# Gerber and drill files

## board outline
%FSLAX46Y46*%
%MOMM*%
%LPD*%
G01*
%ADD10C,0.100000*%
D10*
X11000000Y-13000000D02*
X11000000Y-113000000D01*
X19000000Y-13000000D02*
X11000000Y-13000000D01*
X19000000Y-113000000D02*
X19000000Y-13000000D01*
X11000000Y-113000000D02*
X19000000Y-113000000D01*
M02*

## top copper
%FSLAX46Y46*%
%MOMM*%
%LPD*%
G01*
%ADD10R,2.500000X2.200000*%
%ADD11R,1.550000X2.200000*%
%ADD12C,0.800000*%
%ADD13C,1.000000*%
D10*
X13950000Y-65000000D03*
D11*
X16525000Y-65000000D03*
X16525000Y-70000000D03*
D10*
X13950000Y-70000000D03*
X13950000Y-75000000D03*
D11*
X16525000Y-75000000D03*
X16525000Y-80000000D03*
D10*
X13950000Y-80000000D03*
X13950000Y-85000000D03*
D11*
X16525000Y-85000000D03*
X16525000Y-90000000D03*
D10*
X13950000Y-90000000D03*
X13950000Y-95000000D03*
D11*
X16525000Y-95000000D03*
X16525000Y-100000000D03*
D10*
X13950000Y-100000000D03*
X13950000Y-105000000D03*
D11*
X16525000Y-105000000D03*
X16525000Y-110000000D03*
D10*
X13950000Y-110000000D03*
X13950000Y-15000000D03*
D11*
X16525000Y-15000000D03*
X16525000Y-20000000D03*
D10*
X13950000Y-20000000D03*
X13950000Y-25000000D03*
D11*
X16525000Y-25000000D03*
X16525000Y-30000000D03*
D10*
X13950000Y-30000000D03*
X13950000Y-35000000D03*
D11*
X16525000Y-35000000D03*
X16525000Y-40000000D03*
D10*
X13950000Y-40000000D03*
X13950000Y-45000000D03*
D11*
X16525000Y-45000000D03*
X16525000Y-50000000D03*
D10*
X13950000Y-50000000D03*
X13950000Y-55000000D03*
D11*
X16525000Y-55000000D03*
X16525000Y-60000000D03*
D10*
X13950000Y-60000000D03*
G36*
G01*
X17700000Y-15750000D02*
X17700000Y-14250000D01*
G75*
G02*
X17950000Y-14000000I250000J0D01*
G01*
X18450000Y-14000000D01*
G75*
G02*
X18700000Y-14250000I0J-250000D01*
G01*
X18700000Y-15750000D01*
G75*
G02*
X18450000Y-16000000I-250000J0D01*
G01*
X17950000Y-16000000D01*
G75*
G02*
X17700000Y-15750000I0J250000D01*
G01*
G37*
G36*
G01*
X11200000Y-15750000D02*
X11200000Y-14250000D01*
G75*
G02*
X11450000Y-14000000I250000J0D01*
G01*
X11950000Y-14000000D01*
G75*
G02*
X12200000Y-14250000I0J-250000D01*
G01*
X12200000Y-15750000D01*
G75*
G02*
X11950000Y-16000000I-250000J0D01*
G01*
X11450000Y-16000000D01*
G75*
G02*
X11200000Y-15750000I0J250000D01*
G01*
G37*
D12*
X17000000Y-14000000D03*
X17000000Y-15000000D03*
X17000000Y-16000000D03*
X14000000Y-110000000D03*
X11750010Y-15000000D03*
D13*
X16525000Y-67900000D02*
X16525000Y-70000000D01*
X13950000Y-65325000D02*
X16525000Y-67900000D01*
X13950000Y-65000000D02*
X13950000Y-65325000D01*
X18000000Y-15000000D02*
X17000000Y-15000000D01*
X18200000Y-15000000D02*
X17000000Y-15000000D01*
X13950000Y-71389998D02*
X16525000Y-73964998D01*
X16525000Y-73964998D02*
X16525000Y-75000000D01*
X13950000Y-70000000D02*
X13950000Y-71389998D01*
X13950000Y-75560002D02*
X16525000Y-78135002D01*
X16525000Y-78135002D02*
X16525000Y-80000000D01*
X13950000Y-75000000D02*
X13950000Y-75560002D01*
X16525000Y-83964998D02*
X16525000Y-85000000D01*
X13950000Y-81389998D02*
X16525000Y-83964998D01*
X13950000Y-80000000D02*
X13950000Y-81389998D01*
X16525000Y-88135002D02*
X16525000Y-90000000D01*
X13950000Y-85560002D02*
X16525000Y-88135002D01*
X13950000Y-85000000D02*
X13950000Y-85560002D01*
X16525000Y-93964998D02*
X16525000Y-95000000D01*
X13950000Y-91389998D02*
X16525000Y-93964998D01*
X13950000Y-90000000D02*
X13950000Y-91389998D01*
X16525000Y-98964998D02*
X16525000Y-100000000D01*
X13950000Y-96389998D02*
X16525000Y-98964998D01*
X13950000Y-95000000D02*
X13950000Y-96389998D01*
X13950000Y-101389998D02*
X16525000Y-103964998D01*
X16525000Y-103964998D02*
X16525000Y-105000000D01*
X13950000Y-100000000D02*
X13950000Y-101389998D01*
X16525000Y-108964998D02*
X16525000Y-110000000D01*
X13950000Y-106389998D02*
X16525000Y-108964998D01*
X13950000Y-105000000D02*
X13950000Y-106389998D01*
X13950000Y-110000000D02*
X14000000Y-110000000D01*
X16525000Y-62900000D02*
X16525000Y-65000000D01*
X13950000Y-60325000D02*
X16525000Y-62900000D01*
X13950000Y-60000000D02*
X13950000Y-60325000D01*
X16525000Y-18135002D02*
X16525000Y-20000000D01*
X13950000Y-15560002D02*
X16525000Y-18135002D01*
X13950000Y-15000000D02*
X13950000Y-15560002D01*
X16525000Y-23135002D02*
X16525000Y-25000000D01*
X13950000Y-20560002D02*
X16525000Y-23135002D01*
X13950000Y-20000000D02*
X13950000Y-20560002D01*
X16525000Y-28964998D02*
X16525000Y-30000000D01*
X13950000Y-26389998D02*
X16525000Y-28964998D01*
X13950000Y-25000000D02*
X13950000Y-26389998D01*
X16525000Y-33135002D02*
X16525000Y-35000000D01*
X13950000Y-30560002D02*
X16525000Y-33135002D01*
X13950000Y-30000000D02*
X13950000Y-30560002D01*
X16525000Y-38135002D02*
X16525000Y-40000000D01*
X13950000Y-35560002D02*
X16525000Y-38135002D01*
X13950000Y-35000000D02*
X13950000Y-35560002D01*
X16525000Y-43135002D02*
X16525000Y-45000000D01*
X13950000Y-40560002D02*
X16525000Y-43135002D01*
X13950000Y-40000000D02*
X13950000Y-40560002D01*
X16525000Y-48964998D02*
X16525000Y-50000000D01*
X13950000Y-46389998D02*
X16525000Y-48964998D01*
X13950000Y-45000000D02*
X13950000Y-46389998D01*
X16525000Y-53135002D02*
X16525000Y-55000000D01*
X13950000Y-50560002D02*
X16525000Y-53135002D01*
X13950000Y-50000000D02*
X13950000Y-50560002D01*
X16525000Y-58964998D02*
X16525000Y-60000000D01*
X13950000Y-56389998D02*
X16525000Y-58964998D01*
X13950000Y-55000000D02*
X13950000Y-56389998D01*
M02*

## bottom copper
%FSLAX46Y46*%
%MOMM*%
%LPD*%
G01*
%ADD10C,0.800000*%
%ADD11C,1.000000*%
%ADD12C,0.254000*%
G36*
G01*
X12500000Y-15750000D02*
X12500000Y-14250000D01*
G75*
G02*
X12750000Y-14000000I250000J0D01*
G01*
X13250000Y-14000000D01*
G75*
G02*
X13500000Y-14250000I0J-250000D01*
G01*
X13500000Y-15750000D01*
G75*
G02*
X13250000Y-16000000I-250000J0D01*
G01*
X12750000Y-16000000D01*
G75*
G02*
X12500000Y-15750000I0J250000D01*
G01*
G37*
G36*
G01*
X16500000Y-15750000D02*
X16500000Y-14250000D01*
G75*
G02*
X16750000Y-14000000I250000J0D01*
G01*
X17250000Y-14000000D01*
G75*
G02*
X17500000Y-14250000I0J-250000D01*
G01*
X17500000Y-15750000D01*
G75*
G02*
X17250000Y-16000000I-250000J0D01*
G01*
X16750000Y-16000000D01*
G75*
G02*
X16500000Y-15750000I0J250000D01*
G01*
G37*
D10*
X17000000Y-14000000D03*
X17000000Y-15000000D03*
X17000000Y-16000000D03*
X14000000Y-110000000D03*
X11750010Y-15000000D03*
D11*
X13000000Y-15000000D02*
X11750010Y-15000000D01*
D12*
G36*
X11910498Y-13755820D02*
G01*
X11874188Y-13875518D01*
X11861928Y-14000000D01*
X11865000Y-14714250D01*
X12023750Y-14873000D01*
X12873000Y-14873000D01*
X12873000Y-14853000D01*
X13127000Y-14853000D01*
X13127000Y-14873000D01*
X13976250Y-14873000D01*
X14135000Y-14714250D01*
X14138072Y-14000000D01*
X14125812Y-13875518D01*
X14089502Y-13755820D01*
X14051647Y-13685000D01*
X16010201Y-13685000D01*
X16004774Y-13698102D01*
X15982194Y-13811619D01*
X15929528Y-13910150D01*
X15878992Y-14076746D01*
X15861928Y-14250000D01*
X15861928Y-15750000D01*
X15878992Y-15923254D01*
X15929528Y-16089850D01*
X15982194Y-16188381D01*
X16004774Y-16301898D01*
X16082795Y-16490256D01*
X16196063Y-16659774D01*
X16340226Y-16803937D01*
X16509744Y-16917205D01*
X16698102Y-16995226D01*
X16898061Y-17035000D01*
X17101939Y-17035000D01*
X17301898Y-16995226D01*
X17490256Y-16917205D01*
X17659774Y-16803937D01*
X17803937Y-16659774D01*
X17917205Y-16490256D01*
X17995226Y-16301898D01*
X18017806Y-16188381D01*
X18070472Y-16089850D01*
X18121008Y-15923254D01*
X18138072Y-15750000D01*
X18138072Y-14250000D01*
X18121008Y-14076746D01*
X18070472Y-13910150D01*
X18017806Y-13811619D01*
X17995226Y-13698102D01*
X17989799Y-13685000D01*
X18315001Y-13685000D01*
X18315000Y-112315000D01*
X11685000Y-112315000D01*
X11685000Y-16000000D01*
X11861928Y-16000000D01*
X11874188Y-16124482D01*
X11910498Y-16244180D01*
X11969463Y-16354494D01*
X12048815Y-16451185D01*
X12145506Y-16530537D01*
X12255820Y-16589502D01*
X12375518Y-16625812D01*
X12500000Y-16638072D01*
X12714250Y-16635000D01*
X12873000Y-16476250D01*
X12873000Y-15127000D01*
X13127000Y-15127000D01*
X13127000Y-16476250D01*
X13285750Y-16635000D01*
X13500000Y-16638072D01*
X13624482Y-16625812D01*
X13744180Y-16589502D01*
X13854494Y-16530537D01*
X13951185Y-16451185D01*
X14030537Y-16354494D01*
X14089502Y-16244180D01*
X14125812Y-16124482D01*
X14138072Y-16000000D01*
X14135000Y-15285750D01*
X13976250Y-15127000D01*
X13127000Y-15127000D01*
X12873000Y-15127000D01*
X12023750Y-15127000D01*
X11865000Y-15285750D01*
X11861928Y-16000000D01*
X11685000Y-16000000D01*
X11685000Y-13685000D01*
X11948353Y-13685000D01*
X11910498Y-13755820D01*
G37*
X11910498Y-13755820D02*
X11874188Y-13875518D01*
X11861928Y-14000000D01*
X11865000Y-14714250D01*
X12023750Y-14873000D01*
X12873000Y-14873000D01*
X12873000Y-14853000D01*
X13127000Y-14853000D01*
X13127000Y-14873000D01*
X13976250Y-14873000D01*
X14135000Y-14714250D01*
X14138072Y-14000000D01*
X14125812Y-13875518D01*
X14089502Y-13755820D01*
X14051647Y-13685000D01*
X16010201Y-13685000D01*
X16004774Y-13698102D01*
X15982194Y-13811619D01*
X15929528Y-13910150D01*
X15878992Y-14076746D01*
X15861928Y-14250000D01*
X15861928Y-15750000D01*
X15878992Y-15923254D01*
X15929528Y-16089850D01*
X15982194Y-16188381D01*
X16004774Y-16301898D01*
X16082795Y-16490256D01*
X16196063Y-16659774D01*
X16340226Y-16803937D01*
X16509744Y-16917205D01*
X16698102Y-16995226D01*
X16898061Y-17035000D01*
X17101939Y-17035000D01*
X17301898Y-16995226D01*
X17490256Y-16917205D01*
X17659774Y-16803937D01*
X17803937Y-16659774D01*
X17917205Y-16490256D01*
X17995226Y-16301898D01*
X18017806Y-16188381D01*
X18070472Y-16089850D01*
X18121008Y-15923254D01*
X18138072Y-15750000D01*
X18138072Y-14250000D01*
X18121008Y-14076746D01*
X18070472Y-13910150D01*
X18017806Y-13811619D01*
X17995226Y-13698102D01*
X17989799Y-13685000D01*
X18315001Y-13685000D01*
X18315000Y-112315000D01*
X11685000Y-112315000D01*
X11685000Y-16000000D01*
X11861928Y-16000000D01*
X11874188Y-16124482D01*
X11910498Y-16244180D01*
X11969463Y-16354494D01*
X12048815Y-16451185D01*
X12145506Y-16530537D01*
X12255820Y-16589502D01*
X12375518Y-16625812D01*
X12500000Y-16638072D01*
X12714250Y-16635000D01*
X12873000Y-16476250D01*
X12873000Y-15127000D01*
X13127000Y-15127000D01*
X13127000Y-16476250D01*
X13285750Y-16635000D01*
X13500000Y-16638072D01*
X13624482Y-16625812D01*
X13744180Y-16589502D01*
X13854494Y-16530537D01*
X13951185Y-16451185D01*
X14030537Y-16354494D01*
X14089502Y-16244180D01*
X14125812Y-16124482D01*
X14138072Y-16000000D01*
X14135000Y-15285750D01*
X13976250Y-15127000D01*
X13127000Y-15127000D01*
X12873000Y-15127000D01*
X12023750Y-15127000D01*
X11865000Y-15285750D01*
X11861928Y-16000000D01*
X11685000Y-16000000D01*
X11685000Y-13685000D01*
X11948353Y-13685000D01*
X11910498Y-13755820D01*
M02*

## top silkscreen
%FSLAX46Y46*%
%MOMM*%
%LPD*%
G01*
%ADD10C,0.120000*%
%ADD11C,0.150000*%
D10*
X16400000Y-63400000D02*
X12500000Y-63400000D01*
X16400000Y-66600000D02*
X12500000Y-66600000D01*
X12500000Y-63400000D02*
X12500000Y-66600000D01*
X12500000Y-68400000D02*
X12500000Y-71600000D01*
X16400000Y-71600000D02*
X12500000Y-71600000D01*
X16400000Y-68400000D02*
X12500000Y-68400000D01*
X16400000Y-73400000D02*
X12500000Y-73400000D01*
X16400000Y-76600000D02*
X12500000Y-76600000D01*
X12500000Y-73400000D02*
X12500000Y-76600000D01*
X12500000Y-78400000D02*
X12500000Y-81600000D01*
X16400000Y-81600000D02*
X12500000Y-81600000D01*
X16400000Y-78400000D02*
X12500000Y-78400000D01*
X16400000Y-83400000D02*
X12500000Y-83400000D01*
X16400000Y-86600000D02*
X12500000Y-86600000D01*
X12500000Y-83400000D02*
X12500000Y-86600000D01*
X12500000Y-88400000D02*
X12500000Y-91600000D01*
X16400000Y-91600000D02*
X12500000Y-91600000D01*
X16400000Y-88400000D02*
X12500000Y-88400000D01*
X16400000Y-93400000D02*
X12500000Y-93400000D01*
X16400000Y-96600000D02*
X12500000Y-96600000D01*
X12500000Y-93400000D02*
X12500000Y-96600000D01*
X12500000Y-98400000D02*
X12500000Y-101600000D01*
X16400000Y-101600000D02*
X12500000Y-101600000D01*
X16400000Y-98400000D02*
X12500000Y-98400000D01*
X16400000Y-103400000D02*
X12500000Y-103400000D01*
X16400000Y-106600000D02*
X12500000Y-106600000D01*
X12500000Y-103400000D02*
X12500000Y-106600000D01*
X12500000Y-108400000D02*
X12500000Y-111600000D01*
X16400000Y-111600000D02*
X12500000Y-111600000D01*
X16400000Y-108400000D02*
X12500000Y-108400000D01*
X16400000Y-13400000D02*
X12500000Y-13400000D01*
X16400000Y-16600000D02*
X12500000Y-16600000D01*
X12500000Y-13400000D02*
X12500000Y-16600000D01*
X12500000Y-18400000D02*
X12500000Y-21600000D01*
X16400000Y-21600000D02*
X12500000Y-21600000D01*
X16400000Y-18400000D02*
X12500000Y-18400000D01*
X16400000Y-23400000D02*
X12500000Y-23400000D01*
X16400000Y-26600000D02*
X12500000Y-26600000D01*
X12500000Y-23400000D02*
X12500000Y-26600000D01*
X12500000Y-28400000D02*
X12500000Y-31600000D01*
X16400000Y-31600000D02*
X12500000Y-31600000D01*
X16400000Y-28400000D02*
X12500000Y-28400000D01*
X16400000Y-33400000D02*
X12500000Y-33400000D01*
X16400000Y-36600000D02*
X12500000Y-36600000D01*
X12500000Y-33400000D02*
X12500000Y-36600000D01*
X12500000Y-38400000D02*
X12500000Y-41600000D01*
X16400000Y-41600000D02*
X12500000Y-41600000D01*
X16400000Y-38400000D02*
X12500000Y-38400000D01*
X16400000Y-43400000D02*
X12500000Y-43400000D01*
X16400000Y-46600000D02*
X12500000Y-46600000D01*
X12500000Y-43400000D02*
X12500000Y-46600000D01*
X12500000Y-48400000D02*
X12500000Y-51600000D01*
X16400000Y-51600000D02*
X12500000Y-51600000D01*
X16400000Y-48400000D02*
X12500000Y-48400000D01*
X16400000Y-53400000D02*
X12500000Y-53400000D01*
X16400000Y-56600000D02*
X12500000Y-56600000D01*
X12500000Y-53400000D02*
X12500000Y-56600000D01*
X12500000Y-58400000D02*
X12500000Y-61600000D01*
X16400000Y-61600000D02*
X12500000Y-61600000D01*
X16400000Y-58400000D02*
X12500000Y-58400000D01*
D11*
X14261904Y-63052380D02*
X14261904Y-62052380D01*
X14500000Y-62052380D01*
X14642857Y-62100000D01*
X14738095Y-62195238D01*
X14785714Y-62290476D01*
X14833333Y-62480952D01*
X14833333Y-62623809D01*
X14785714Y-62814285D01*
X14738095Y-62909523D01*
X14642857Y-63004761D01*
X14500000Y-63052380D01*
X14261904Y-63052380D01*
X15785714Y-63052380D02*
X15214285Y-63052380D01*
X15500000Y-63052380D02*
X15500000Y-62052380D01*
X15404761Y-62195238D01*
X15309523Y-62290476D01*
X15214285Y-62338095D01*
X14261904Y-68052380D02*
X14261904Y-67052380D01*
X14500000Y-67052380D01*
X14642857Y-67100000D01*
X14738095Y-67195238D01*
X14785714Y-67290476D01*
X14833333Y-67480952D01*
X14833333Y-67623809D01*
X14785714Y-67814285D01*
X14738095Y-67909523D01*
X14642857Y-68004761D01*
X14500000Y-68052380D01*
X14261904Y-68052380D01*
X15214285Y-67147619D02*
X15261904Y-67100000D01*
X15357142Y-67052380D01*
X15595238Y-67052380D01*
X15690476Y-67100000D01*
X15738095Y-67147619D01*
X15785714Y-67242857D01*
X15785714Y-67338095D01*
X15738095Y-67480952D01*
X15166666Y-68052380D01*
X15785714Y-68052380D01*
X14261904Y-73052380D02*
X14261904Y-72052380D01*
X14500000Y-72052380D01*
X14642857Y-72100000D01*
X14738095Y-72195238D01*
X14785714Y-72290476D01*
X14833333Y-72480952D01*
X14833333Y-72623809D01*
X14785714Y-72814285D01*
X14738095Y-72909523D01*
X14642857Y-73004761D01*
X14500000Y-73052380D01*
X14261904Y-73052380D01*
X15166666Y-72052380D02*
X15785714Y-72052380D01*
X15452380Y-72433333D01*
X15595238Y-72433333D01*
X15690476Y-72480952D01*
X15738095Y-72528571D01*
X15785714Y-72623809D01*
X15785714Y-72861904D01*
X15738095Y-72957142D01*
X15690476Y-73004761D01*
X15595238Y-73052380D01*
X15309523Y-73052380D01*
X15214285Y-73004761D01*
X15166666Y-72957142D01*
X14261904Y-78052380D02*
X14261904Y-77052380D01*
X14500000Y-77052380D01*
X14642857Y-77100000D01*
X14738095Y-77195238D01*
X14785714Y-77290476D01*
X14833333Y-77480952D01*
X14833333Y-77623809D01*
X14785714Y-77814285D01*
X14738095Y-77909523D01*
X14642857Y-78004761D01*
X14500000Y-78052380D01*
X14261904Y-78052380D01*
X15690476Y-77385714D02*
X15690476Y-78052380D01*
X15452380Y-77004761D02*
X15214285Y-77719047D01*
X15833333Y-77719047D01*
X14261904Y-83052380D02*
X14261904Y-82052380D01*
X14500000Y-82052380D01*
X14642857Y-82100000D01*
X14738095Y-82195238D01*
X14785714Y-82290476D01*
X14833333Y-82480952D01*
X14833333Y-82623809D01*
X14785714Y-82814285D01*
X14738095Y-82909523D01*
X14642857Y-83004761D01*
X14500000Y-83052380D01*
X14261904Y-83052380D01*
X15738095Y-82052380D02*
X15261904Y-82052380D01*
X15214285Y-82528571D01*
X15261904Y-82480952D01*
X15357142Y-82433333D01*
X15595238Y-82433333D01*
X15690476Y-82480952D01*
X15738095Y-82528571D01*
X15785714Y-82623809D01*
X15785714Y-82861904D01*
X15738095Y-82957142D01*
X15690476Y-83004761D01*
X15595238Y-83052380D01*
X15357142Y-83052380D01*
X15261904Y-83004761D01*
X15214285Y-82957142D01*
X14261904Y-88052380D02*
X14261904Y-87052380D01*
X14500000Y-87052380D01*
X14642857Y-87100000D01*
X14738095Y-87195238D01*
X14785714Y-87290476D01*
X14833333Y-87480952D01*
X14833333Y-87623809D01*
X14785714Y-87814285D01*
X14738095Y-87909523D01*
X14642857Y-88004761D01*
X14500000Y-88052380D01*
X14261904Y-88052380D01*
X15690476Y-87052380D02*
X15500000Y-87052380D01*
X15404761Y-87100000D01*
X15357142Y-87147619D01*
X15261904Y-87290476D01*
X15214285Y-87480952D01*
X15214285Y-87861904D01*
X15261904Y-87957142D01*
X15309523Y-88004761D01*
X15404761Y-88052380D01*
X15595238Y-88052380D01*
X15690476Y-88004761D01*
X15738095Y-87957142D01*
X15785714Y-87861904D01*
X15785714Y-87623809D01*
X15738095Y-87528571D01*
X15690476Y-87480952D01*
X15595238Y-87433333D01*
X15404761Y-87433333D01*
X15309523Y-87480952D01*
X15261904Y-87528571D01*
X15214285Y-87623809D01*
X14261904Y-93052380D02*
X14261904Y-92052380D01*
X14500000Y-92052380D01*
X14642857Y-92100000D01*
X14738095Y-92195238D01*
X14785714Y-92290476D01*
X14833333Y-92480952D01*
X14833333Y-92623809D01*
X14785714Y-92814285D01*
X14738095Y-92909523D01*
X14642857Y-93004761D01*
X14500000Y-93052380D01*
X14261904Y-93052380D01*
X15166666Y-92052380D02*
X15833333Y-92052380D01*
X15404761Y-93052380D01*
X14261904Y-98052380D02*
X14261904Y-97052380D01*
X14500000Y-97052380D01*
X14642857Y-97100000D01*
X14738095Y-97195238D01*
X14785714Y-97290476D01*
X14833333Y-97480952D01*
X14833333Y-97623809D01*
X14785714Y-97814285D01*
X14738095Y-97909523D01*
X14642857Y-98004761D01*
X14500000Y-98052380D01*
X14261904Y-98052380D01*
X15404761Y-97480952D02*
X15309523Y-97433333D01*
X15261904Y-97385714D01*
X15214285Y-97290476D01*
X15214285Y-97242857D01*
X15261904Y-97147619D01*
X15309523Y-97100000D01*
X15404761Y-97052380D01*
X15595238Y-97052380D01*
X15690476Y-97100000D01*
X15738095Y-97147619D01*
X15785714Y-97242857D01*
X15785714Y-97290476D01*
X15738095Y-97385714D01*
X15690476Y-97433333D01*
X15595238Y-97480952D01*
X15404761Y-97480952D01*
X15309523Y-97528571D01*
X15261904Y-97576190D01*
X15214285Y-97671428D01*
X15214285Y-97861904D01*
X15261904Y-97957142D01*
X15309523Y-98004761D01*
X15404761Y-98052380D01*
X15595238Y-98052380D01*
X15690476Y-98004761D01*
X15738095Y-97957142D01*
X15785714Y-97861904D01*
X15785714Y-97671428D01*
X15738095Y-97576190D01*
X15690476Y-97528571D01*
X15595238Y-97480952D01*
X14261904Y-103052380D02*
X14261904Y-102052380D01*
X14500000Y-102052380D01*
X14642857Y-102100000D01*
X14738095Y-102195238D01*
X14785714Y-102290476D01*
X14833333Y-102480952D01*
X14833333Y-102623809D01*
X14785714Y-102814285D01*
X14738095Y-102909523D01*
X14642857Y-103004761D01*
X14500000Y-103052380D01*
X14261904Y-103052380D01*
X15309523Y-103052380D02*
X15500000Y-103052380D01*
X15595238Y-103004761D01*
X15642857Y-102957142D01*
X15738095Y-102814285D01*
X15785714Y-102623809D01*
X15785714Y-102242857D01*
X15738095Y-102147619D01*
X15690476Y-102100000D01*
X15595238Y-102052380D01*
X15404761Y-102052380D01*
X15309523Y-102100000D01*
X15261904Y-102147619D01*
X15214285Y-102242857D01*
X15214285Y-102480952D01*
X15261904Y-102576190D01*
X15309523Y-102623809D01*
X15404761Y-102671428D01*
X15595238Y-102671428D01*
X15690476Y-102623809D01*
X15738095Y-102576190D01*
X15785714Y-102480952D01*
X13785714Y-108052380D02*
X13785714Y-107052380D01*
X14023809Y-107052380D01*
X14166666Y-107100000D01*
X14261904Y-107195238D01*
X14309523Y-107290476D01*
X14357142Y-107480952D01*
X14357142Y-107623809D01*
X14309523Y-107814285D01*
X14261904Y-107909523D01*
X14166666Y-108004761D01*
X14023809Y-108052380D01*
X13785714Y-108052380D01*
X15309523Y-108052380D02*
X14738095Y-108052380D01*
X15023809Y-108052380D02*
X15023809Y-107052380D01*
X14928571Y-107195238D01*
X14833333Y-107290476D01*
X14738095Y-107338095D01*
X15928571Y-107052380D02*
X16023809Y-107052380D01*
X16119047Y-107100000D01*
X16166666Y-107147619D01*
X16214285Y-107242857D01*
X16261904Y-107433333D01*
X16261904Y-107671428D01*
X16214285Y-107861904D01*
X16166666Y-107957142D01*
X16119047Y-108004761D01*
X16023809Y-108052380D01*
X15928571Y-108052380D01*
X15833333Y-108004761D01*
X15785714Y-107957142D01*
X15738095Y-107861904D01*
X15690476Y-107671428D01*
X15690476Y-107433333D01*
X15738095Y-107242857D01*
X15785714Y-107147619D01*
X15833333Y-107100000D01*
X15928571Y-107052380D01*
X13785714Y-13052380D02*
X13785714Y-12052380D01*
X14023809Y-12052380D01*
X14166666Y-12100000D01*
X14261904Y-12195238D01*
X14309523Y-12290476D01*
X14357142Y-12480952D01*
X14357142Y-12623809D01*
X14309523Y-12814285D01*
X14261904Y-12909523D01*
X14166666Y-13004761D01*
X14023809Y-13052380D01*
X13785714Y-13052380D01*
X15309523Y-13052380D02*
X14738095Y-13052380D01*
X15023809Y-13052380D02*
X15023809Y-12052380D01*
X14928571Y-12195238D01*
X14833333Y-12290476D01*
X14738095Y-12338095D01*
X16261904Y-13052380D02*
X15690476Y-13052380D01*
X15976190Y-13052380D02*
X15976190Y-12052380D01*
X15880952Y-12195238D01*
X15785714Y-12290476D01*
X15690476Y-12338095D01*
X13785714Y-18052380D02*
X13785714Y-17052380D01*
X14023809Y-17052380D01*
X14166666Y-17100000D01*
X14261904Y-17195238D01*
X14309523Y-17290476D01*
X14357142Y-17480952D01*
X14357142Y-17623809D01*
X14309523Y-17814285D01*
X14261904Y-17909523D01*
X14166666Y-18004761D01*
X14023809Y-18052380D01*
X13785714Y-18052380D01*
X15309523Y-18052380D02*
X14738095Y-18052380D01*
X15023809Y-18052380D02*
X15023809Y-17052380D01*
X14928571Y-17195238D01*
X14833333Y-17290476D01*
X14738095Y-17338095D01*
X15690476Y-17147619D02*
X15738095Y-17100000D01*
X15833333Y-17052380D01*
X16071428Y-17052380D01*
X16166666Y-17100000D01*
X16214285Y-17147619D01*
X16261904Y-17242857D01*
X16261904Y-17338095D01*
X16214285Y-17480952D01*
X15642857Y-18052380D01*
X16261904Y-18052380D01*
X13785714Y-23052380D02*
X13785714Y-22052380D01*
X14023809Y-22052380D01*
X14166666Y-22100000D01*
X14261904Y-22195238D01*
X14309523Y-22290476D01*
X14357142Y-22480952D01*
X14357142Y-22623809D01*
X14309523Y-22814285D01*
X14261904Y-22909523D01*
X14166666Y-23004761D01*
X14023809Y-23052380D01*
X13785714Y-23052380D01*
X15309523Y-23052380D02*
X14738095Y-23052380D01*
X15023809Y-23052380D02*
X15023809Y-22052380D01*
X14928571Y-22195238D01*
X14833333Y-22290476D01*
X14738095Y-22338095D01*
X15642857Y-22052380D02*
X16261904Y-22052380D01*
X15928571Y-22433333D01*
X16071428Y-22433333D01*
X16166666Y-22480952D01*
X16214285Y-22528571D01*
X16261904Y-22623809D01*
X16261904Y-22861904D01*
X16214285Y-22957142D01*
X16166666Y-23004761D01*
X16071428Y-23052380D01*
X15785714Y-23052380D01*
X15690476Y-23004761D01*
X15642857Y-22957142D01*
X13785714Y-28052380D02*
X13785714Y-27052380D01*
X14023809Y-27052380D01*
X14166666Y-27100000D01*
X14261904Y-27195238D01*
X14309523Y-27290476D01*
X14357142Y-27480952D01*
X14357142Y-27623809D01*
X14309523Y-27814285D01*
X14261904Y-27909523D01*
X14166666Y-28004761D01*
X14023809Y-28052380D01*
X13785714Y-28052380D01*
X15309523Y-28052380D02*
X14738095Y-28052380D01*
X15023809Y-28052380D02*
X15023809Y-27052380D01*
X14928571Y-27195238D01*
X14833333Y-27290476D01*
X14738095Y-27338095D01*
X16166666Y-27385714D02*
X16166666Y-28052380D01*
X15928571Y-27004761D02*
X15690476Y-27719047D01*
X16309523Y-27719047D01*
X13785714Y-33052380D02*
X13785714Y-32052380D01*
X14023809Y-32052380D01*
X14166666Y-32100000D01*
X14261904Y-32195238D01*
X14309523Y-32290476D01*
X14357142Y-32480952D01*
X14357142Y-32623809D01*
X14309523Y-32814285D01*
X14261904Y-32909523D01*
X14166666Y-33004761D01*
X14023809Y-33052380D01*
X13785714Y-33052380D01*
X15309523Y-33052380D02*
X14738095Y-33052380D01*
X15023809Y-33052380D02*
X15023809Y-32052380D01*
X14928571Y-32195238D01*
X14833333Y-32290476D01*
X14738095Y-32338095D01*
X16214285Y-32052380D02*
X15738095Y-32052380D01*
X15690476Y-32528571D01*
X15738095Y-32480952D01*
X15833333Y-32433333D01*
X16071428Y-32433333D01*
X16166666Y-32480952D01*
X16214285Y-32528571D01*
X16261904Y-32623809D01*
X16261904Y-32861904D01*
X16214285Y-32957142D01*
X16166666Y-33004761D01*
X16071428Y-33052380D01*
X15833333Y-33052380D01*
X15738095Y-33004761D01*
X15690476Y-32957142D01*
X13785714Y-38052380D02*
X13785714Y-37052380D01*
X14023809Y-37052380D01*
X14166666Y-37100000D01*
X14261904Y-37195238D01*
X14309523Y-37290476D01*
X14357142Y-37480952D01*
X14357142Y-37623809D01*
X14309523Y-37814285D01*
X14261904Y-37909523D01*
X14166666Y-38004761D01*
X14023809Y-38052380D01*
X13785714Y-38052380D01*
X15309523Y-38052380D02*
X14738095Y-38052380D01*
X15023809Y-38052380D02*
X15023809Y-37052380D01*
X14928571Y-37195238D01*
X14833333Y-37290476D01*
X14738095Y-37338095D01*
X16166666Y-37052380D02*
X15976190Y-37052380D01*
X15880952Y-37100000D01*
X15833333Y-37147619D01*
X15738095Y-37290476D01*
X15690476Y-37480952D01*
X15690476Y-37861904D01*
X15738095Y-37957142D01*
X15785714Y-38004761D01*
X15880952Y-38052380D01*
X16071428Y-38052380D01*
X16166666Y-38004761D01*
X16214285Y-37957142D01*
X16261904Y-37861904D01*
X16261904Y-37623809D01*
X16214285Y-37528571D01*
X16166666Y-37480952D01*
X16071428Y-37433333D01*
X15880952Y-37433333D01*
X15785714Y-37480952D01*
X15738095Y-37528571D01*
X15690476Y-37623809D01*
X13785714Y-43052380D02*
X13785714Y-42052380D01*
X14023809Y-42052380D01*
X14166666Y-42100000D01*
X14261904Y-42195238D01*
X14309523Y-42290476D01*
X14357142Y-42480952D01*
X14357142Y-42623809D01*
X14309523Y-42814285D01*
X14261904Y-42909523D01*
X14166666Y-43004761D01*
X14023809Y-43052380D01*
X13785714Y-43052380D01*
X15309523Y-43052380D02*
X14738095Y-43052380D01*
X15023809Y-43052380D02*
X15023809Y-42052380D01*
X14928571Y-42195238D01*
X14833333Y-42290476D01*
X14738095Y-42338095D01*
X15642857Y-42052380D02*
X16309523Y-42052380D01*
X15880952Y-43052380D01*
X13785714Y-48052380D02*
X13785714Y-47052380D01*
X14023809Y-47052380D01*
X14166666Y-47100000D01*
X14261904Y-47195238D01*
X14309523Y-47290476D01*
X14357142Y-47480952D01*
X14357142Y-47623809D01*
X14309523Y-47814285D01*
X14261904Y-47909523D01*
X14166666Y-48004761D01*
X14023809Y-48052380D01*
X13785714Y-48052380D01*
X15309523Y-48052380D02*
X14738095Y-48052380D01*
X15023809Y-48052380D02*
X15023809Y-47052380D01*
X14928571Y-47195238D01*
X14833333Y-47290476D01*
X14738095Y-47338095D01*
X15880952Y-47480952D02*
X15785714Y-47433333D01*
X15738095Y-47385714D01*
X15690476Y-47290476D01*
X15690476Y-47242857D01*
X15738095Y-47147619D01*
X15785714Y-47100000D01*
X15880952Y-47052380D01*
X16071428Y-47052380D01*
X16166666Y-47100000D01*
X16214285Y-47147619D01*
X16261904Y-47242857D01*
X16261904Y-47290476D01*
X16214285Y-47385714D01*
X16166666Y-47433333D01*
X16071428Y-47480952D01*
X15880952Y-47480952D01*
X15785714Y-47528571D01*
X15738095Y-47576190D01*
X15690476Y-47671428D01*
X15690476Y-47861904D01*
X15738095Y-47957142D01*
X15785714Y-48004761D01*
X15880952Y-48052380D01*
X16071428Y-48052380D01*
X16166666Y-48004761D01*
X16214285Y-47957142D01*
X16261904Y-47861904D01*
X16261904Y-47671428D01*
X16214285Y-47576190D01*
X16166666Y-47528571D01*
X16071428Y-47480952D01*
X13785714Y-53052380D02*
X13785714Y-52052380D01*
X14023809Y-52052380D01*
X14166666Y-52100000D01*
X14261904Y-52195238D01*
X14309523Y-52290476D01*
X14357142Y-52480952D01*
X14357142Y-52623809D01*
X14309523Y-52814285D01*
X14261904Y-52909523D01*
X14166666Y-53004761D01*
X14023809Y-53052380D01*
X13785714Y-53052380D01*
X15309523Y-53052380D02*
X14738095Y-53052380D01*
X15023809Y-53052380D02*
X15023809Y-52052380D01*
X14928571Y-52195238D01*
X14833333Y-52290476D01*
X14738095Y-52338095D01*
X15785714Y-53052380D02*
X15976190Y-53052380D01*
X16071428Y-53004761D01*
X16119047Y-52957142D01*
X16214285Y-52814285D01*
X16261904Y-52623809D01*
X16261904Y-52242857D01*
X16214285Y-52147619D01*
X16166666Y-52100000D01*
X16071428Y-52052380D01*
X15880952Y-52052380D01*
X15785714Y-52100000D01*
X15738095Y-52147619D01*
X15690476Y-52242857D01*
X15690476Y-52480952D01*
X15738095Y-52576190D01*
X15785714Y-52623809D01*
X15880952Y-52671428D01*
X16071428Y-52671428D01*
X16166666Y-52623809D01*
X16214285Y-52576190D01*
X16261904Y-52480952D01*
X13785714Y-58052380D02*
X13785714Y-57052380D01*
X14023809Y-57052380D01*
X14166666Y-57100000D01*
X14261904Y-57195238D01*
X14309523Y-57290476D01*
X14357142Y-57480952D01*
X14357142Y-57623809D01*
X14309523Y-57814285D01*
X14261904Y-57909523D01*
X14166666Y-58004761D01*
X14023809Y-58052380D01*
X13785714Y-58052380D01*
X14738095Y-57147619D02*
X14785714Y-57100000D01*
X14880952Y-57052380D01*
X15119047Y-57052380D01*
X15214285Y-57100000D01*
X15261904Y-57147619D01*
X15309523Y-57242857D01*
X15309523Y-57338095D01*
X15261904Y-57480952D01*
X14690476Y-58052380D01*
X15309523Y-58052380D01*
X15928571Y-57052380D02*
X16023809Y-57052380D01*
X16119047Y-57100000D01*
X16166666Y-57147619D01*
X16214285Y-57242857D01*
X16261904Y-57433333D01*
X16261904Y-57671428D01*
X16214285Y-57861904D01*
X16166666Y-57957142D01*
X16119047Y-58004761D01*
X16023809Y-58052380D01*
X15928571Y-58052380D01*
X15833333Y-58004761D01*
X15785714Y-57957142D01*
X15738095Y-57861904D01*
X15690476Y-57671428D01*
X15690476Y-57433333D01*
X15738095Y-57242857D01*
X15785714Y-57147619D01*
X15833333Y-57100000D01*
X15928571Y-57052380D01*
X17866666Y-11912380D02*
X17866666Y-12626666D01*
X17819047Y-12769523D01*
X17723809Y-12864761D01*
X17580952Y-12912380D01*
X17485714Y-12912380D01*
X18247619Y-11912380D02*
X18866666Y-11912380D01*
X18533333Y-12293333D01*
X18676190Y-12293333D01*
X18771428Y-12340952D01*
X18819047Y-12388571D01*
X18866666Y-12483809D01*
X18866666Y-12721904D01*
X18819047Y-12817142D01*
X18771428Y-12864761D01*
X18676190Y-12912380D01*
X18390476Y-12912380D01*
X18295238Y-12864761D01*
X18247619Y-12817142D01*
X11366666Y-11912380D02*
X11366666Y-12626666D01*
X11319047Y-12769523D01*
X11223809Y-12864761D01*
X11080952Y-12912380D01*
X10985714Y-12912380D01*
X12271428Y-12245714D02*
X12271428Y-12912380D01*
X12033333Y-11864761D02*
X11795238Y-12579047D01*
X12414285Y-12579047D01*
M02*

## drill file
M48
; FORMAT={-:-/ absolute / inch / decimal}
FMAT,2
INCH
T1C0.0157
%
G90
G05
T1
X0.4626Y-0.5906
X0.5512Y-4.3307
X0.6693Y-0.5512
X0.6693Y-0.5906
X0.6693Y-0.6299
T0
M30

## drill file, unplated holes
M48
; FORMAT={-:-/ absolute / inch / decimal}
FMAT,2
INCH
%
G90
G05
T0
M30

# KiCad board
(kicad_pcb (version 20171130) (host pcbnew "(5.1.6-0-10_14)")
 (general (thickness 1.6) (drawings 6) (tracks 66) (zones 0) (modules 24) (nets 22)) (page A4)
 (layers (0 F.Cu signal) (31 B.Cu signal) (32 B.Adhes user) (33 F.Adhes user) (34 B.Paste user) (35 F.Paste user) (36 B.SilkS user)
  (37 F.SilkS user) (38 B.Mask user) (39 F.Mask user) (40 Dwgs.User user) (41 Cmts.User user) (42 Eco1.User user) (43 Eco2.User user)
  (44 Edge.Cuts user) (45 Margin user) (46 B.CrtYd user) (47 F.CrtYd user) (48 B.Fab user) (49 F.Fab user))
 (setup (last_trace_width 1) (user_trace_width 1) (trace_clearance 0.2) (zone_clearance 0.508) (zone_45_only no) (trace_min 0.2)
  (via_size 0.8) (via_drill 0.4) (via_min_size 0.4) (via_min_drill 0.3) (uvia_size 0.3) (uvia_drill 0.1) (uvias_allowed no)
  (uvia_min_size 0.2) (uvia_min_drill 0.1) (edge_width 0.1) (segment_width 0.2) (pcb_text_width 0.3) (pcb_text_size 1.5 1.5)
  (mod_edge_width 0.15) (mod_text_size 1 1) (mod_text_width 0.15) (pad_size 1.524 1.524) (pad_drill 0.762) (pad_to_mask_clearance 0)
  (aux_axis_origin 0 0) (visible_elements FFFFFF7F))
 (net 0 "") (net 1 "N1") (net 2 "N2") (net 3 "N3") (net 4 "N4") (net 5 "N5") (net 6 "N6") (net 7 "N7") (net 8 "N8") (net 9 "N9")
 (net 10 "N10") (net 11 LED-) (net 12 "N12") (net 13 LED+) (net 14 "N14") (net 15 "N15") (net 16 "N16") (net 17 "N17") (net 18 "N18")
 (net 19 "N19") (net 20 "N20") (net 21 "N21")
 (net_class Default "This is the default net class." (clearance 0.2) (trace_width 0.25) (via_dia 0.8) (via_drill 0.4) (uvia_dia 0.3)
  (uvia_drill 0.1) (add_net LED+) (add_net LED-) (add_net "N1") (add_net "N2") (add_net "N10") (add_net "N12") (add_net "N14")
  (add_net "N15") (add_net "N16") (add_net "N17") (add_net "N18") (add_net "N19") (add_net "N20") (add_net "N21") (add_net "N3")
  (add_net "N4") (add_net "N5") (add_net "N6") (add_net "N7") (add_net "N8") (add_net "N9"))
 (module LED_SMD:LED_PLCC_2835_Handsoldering (layer F.Cu) (at 15 65)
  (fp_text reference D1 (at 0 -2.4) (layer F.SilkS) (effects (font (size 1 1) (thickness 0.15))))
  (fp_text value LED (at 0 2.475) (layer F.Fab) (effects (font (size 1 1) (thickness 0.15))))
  (fp_line (start 1.4 -1.6) (end -2.5 -1.6) (layer F.SilkS) (width 0.12))
  (fp_line (start 1.4 1.6) (end -2.5 1.6) (layer F.SilkS) (width 0.12))
  (fp_line (start -2.5 -1.6) (end -2.5 1.6) (layer F.SilkS) (width 0.12))
  (pad 1 smd rect (at -1.05 0) (size 2.5 2.2) (layers F.Cu F.Paste F.Mask) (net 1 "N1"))
  (pad 2 smd rect (at 1.525 0) (size 1.55 2.2) (layers F.Cu F.Paste F.Mask) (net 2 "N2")))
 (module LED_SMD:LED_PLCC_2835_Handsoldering (layer F.Cu) (at 15 70)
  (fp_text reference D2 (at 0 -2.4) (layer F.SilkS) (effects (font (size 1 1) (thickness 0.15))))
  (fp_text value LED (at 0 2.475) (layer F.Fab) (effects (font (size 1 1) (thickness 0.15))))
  (fp_line (start -2.5 -1.6) (end -2.5 1.6) (layer F.SilkS) (width 0.12))
  (fp_line (start 1.4 1.6) (end -2.5 1.6) (layer F.SilkS) (width 0.12))
  (fp_line (start 1.4 -1.6) (end -2.5 -1.6) (layer F.SilkS) (width 0.12))
  (pad 2 smd rect (at 1.525 0) (size 1.55 2.2) (layers F.Cu F.Paste F.Mask) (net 1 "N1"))
  (pad 1 smd rect (at -1.05 0) (size 2.5 2.2) (layers F.Cu F.Paste F.Mask) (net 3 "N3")))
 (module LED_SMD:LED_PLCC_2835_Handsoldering (layer F.Cu) (at 15 75)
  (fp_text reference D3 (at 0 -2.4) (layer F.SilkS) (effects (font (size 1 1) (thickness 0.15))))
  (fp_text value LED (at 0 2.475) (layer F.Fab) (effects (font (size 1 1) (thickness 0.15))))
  (fp_line (start 1.4 -1.6) (end -2.5 -1.6) (layer F.SilkS) (width 0.12))
  (fp_line (start 1.4 1.6) (end -2.5 1.6) (layer F.SilkS) (width 0.12))
  (fp_line (start -2.5 -1.6) (end -2.5 1.6) (layer F.SilkS) (width 0.12))
  (pad 1 smd rect (at -1.05 0) (size 2.5 2.2) (layers F.Cu F.Paste F.Mask) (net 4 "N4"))
  (pad 2 smd rect (at 1.525 0) (size 1.55 2.2) (layers F.Cu F.Paste F.Mask) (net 3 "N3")))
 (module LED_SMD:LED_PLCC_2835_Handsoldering (layer F.Cu) (at 15 80)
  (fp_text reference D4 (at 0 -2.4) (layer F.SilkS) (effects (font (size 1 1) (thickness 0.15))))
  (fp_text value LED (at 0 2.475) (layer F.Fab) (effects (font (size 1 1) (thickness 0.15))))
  (fp_line (start -2.5 -1.6) (end -2.5 1.6) (layer F.SilkS) (width 0.12))
  (fp_line (start 1.4 1.6) (end -2.5 1.6) (layer F.SilkS) (width 0.12))
  (fp_line (start 1.4 -1.6) (end -2.5 -1.6) (layer F.SilkS) (width 0.12))
  (pad 2 smd rect (at 1.525 0) (size 1.55 2.2) (layers F.Cu F.Paste F.Mask) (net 4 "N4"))
  (pad 1 smd rect (at -1.05 0) (size 2.5 2.2) (layers F.Cu F.Paste F.Mask) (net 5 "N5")))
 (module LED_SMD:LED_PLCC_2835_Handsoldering (layer F.Cu) (at 15 85)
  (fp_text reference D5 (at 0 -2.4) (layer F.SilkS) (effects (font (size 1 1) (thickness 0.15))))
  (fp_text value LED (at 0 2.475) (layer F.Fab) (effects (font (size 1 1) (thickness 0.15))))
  (fp_line (start 1.4 -1.6) (end -2.5 -1.6) (layer F.SilkS) (width 0.12))
  (fp_line (start 1.4 1.6) (end -2.5 1.6) (layer F.SilkS) (width 0.12))
  (fp_line (start -2.5 -1.6) (end -2.5 1.6) (layer F.SilkS) (width 0.12))
  (pad 1 smd rect (at -1.05 0) (size 2.5 2.2) (layers F.Cu F.Paste F.Mask) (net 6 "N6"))
  (pad 2 smd rect (at 1.525 0) (size 1.55 2.2) (layers F.Cu F.Paste F.Mask) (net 5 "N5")))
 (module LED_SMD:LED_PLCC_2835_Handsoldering (layer F.Cu) (at 15 90)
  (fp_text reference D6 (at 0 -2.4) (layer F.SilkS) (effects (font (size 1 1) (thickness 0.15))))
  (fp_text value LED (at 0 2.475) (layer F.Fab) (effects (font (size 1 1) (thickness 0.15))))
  (fp_line (start -2.5 -1.6) (end -2.5 1.6) (layer F.SilkS) (width 0.12))
  (fp_line (start 1.4 1.6) (end -2.5 1.6) (layer F.SilkS) (width 0.12))
  (fp_line (start 1.4 -1.6) (end -2.5 -1.6) (layer F.SilkS) (width 0.12))
  (pad 2 smd rect (at 1.525 0) (size 1.55 2.2) (layers F.Cu F.Paste F.Mask) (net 6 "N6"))
  (pad 1 smd rect (at -1.05 0) (size 2.5 2.2) (layers F.Cu F.Paste F.Mask) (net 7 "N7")))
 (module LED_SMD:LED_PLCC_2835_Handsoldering (layer F.Cu) (at 15 95)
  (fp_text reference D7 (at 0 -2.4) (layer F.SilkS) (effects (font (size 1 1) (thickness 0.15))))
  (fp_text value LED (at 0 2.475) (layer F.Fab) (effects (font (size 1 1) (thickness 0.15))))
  (fp_line (start 1.4 -1.6) (end -2.5 -1.6) (layer F.SilkS) (width 0.12))
  (fp_line (start 1.4 1.6) (end -2.5 1.6) (layer F.SilkS) (width 0.12))
  (fp_line (start -2.5 -1.6) (end -2.5 1.6) (layer F.SilkS) (width 0.12))
  (pad 1 smd rect (at -1.05 0) (size 2.5 2.2) (layers F.Cu F.Paste F.Mask) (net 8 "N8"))
  (pad 2 smd rect (at 1.525 0) (size 1.55 2.2) (layers F.Cu F.Paste F.Mask) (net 7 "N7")))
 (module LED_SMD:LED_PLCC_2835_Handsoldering (layer F.Cu) (at 15 100)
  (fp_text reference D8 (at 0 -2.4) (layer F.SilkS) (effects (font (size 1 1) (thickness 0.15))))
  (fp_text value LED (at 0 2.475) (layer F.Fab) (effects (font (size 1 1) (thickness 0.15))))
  (fp_line (start -2.5 -1.6) (end -2.5 1.6) (layer F.SilkS) (width 0.12))
  (fp_line (start 1.4 1.6) (end -2.5 1.6) (layer F.SilkS) (width 0.12))
  (fp_line (start 1.4 -1.6) (end -2.5 -1.6) (layer F.SilkS) (width 0.12))
  (pad 2 smd rect (at 1.525 0) (size 1.55 2.2) (layers F.Cu F.Paste F.Mask) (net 8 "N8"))
  (pad 1 smd rect (at -1.05 0) (size 2.5 2.2) (layers F.Cu F.Paste F.Mask) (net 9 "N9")))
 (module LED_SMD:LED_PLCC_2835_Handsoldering (layer F.Cu) (at 15 105)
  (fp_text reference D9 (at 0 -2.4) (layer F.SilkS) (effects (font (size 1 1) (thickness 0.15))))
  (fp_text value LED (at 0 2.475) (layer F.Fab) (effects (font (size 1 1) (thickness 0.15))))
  (fp_line (start 1.4 -1.6) (end -2.5 -1.6) (layer F.SilkS) (width 0.12))
  (fp_line (start 1.4 1.6) (end -2.5 1.6) (layer F.SilkS) (width 0.12))
  (fp_line (start -2.5 -1.6) (end -2.5 1.6) (layer F.SilkS) (width 0.12))
  (pad 1 smd rect (at -1.05 0) (size 2.5 2.2) (layers F.Cu F.Paste F.Mask) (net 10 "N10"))
  (pad 2 smd rect (at 1.525 0) (size 1.55 2.2) (layers F.Cu F.Paste F.Mask) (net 9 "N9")))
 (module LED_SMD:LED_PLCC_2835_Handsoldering (layer F.Cu) (at 15 110)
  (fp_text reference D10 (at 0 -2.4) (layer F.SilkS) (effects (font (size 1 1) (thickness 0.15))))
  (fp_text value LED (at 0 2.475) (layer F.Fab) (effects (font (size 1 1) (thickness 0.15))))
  (fp_line (start -2.5 -1.6) (end -2.5 1.6) (layer F.SilkS) (width 0.12))
  (fp_line (start 1.4 1.6) (end -2.5 1.6) (layer F.SilkS) (width 0.12))
  (fp_line (start 1.4 -1.6) (end -2.5 -1.6) (layer F.SilkS) (width 0.12))
  (pad 2 smd rect (at 1.525 0) (size 1.55 2.2) (layers F.Cu F.Paste F.Mask) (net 10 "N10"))
  (pad 1 smd rect (at -1.05 0) (size 2.5 2.2) (layers F.Cu F.Paste F.Mask) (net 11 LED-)))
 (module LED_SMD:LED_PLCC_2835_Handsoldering (layer F.Cu) (at 15 15)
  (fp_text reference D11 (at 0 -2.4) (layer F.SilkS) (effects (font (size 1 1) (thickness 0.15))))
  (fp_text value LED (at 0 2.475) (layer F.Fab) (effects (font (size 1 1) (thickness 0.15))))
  (fp_line (start 1.4 -1.6) (end -2.5 -1.6) (layer F.SilkS) (width 0.12))
  (fp_line (start 1.4 1.6) (end -2.5 1.6) (layer F.SilkS) (width 0.12))
  (fp_line (start -2.5 -1.6) (end -2.5 1.6) (layer F.SilkS) (width 0.12))
  (pad 1 smd rect (at -1.05 0) (size 2.5 2.2) (layers F.Cu F.Paste F.Mask) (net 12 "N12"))
  (pad 2 smd rect (at 1.525 0) (size 1.55 2.2) (layers F.Cu F.Paste F.Mask) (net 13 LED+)))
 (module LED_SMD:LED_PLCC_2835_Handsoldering (layer F.Cu) (at 15 20)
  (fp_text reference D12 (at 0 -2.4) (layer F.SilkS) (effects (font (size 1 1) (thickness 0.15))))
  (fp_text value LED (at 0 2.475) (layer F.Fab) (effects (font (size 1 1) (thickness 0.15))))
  (fp_line (start -2.5 -1.6) (end -2.5 1.6) (layer F.SilkS) (width 0.12))
  (fp_line (start 1.4 1.6) (end -2.5 1.6) (layer F.SilkS) (width 0.12))
  (fp_line (start 1.4 -1.6) (end -2.5 -1.6) (layer F.SilkS) (width 0.12))
  (pad 2 smd rect (at 1.525 0) (size 1.55 2.2) (layers F.Cu F.Paste F.Mask) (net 12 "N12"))
  (pad 1 smd rect (at -1.05 0) (size 2.5 2.2) (layers F.Cu F.Paste F.Mask) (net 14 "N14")))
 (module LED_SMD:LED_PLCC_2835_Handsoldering (layer F.Cu) (at 15 25)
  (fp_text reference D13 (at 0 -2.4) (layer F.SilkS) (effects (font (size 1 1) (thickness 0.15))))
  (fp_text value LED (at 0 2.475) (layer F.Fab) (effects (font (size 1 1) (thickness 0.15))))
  (fp_line (start 1.4 -1.6) (end -2.5 -1.6) (layer F.SilkS) (width 0.12))
  (fp_line (start 1.4 1.6) (end -2.5 1.6) (layer F.SilkS) (width 0.12))
  (fp_line (start -2.5 -1.6) (end -2.5 1.6) (layer F.SilkS) (width 0.12))
  (pad 1 smd rect (at -1.05 0) (size 2.5 2.2) (layers F.Cu F.Paste F.Mask) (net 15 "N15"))
  (pad 2 smd rect (at 1.525 0) (size 1.55 2.2) (layers F.Cu F.Paste F.Mask) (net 14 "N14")))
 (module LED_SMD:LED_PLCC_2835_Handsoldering (layer F.Cu) (at 15 30)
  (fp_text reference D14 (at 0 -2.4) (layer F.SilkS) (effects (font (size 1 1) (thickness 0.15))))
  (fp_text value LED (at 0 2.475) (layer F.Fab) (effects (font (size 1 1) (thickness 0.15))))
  (fp_line (start -2.5 -1.6) (end -2.5 1.6) (layer F.SilkS) (width 0.12))
  (fp_line (start 1.4 1.6) (end -2.5 1.6) (layer F.SilkS) (width 0.12))
  (fp_line (start 1.4 -1.6) (end -2.5 -1.6) (layer F.SilkS) (width 0.12))
  (pad 2 smd rect (at 1.525 0) (size 1.55 2.2) (layers F.Cu F.Paste F.Mask) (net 15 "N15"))
  (pad 1 smd rect (at -1.05 0) (size 2.5 2.2) (layers F.Cu F.Paste F.Mask) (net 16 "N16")))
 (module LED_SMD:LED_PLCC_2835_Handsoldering (layer F.Cu) (at 15 35)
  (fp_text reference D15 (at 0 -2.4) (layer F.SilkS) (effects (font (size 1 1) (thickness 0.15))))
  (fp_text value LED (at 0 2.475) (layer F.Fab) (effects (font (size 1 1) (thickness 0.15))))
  (fp_line (start 1.4 -1.6) (end -2.5 -1.6) (layer F.SilkS) (width 0.12))
  (fp_line (start 1.4 1.6) (end -2.5 1.6) (layer F.SilkS) (width 0.12))
  (fp_line (start -2.5 -1.6) (end -2.5 1.6) (layer F.SilkS) (width 0.12))
  (pad 1 smd rect (at -1.05 0) (size 2.5 2.2) (layers F.Cu F.Paste F.Mask) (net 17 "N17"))
  (pad 2 smd rect (at 1.525 0) (size 1.55 2.2) (layers F.Cu F.Paste F.Mask) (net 16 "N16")))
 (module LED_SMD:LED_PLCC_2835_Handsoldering (layer F.Cu) (at 15 40)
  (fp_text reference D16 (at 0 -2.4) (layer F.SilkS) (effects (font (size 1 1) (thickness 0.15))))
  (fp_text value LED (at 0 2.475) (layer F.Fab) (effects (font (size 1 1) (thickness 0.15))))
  (fp_line (start -2.5 -1.6) (end -2.5 1.6) (layer F.SilkS) (width 0.12))
  (fp_line (start 1.4 1.6) (end -2.5 1.6) (layer F.SilkS) (width 0.12))
  (fp_line (start 1.4 -1.6) (end -2.5 -1.6) (layer F.SilkS) (width 0.12))
  (pad 2 smd rect (at 1.525 0) (size 1.55 2.2) (layers F.Cu F.Paste F.Mask) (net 17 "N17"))
  (pad 1 smd rect (at -1.05 0) (size 2.5 2.2) (layers F.Cu F.Paste F.Mask) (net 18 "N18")))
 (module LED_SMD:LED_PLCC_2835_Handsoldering (layer F.Cu) (at 15 45)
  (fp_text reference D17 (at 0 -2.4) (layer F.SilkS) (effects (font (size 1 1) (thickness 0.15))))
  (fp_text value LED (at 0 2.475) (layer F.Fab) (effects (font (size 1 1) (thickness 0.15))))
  (fp_line (start 1.4 -1.6) (end -2.5 -1.6) (layer F.SilkS) (width 0.12))
  (fp_line (start 1.4 1.6) (end -2.5 1.6) (layer F.SilkS) (width 0.12))
  (fp_line (start -2.5 -1.6) (end -2.5 1.6) (layer F.SilkS) (width 0.12))
  (pad 1 smd rect (at -1.05 0) (size 2.5 2.2) (layers F.Cu F.Paste F.Mask) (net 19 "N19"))
  (pad 2 smd rect (at 1.525 0) (size 1.55 2.2) (layers F.Cu F.Paste F.Mask) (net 18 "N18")))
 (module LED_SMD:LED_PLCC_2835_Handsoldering (layer F.Cu) (at 15 50)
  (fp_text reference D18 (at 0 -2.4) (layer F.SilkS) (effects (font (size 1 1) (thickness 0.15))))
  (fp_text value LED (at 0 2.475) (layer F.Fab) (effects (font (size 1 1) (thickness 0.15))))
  (fp_line (start -2.5 -1.6) (end -2.5 1.6) (layer F.SilkS) (width 0.12))
  (fp_line (start 1.4 1.6) (end -2.5 1.6) (layer F.SilkS) (width 0.12))
  (fp_line (start 1.4 -1.6) (end -2.5 -1.6) (layer F.SilkS) (width 0.12))
  (pad 2 smd rect (at 1.525 0) (size 1.55 2.2) (layers F.Cu F.Paste F.Mask) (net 19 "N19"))
  (pad 1 smd rect (at -1.05 0) (size 2.5 2.2) (layers F.Cu F.Paste F.Mask) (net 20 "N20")))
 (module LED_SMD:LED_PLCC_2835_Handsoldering (layer F.Cu) (at 15 55)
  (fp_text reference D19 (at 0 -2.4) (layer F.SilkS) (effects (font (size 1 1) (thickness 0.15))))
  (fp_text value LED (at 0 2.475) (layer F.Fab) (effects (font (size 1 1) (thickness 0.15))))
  (fp_line (start 1.4 -1.6) (end -2.5 -1.6) (layer F.SilkS) (width 0.12))
  (fp_line (start 1.4 1.6) (end -2.5 1.6) (layer F.SilkS) (width 0.12))
  (fp_line (start -2.5 -1.6) (end -2.5 1.6) (layer F.SilkS) (width 0.12))
  (pad 1 smd rect (at -1.05 0) (size 2.5 2.2) (layers F.Cu F.Paste F.Mask) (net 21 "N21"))
  (pad 2 smd rect (at 1.525 0) (size 1.55 2.2) (layers F.Cu F.Paste F.Mask) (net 20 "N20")))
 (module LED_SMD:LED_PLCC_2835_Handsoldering (layer F.Cu) (at 15 60)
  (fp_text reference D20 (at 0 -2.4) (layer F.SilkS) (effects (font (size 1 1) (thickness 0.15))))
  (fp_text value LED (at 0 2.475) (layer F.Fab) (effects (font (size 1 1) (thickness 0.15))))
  (fp_line (start -2.5 -1.6) (end -2.5 1.6) (layer F.SilkS) (width 0.12))
  (fp_line (start 1.4 1.6) (end -2.5 1.6) (layer F.SilkS) (width 0.12))
  (fp_line (start 1.4 -1.6) (end -2.5 -1.6) (layer F.SilkS) (width 0.12))
  (pad 2 smd rect (at 1.525 0) (size 1.55 2.2) (layers F.Cu F.Paste F.Mask) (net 21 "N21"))
  (pad 1 smd rect (at -1.05 0) (size 2.5 2.2) (layers F.Cu F.Paste F.Mask) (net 2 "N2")))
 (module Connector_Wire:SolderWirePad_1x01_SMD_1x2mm (layer B.Cu) (at 13 15)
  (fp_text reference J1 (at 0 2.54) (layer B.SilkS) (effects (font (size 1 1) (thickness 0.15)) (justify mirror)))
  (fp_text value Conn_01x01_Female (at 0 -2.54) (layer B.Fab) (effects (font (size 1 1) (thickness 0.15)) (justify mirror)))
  (pad 1 smd roundrect (at 0 0) (size 1 2) (layers B.Cu B.Paste B.Mask) (roundrect_rratio 0.25) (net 11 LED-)))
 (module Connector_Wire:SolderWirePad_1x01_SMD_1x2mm (layer B.Cu) (at 17 15)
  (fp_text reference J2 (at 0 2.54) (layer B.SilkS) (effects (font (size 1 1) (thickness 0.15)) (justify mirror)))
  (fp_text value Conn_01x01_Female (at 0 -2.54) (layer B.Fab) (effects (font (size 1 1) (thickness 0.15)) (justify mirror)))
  (pad 1 smd roundrect (at 0 0) (size 1 2) (layers B.Cu B.Paste B.Mask) (roundrect_rratio 0.25) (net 13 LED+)))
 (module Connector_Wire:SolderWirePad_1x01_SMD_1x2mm (layer F.Cu) (at 18.2 15)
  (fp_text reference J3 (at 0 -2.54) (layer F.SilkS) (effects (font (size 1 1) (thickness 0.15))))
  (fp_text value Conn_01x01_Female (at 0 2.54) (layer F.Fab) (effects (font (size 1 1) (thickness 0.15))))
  (pad 1 smd roundrect (at 0 0) (size 1 2) (layers F.Cu F.Paste F.Mask) (roundrect_rratio 0.25) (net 13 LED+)))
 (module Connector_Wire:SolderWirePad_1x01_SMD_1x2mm (layer F.Cu) (at 11.7 15)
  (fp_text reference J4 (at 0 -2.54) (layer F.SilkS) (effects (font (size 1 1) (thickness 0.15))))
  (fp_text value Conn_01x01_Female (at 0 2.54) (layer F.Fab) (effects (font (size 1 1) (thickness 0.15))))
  (pad 1 smd roundrect (at 0 0) (size 1 2) (layers F.Cu F.Paste F.Mask) (roundrect_rratio 0.25) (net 11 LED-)))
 (gr_line (start 11 13) (end 11 113) (layer Edge.Cuts) (width 0.1))
 (gr_line (start 19 13) (end 11 13) (layer Edge.Cuts) (width 0.1))
 (gr_line (start 19 113) (end 19 13) (layer Edge.Cuts) (width 0.1))
 (gr_line (start 11 113) (end 19 113) (layer Edge.Cuts) (width 0.1))
 (segment (start 16.525 67.9) (end 16.525 70) (width 1) (layer F.Cu) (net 1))
 (segment (start 13.95 65.325) (end 16.525 67.9) (width 1) (layer F.Cu) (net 1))
 (segment (start 13.95 65) (end 13.95 65.325) (width 1) (layer F.Cu) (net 1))
 (via (at 17 14) (size 0.8) (drill 0.4) (layers F.Cu B.Cu) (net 13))
 (via (at 17 15) (size 0.8) (drill 0.4) (layers F.Cu B.Cu) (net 13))
 (via (at 17 16) (size 0.8) (drill 0.4) (layers F.Cu B.Cu) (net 13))
 (segment (start 18 15) (end 17 15) (width 1) (layer F.Cu) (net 13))
 (segment (start 18.2 15) (end 17 15) (width 1) (layer F.Cu) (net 13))
 (segment (start 13.95 71.389998) (end 16.525 73.964998) (width 1) (layer F.Cu) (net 3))
 (segment (start 16.525 73.964998) (end 16.525 75) (width 1) (layer F.Cu) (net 3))
 (segment (start 13.95 70) (end 13.95 71.389998) (width 1) (layer F.Cu) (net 3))
 (segment (start 13.95 75.560002) (end 16.525 78.135002) (width 1) (layer F.Cu) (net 4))
 (segment (start 16.525 78.135002) (end 16.525 80) (width 1) (layer F.Cu) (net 4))
 (segment (start 13.95 75) (end 13.95 75.560002) (width 1) (layer F.Cu) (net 4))
 (segment (start 16.525 83.964998) (end 16.525 85) (width 1) (layer F.Cu) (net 5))
 (segment (start 13.95 81.389998) (end 16.525 83.964998) (width 1) (layer F.Cu) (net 5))
 (segment (start 13.95 80) (end 13.95 81.389998) (width 1) (layer F.Cu) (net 5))
 (segment (start 16.525 88.135002) (end 16.525 90) (width 1) (layer F.Cu) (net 6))
 (segment (start 13.95 85.560002) (end 16.525 88.135002) (width 1) (layer F.Cu) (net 6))
 (segment (start 13.95 85) (end 13.95 85.560002) (width 1) (layer F.Cu) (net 6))
 (segment (start 16.525 93.964998) (end 16.525 95) (width 1) (layer F.Cu) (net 7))
 (segment (start 13.95 91.389998) (end 16.525 93.964998) (width 1) (layer F.Cu) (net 7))
 (segment (start 13.95 90) (end 13.95 91.389998) (width 1) (layer F.Cu) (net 7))
 (segment (start 16.525 98.964998) (end 16.525 100) (width 1) (layer F.Cu) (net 8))
 (segment (start 13.95 96.389998) (end 16.525 98.964998) (width 1) (layer F.Cu) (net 8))
 (segment (start 13.95 95) (end 13.95 96.389998) (width 1) (layer F.Cu) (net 8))
 (segment (start 13.95 101.389998) (end 16.525 103.964998) (width 1) (layer F.Cu) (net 9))
 (segment (start 16.525 103.964998) (end 16.525 105) (width 1) (layer F.Cu) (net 9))
 (segment (start 13.95 100) (end 13.95 101.389998) (width 1) (layer F.Cu) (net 9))
 (segment (start 16.525 108.964998) (end 16.525 110) (width 1) (layer F.Cu) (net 10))
 (segment (start 13.95 106.389998) (end 16.525 108.964998) (width 1) (layer F.Cu) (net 10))
 (segment (start 13.95 105) (end 13.95 106.389998) (width 1) (layer F.Cu) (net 10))
 (via (at 14 110) (size 0.8) (drill 0.4) (layers F.Cu B.Cu) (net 11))
 (segment (start 13.95 110) (end 14 110) (width 1) (layer F.Cu) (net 11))
 (segment (start 13 15) (end 11.75001 15) (width 1) (layer B.Cu) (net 11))
 (via (at 11.75001 15) (size 0.8) (drill 0.4) (layers F.Cu B.Cu) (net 11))
 (segment (start 16.525 62.9) (end 16.525 65) (width 1) (layer F.Cu) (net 2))
 (segment (start 13.95 60.325) (end 16.525 62.9) (width 1) (layer F.Cu) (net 2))
 (segment (start 13.95 60) (end 13.95 60.325) (width 1) (layer F.Cu) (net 2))
 (segment (start 16.525 18.135002) (end 16.525 20) (width 1) (layer F.Cu) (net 12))
 (segment (start 13.95 15.560002) (end 16.525 18.135002) (width 1) (layer F.Cu) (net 12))
 (segment (start 13.95 15) (end 13.95 15.560002) (width 1) (layer F.Cu) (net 12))
 (segment (start 16.525 23.135002) (end 16.525 25) (width 1) (layer F.Cu) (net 14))
 (segment (start 13.95 20.560002) (end 16.525 23.135002) (width 1) (layer F.Cu) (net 14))
 (segment (start 13.95 20) (end 13.95 20.560002) (width 1) (layer F.Cu) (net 14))
 (segment (start 16.525 28.964998) (end 16.525 30) (width 1) (layer F.Cu) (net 15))
 (segment (start 13.95 26.389998) (end 16.525 28.964998) (width 1) (layer F.Cu) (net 15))
 (segment (start 13.95 25) (end 13.95 26.389998) (width 1) (layer F.Cu) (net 15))
 (segment (start 16.525 33.135002) (end 16.525 35) (width 1) (layer F.Cu) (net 16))
 (segment (start 13.95 30.560002) (end 16.525 33.135002) (width 1) (layer F.Cu) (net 16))
 (segment (start 13.95 30) (end 13.95 30.560002) (width 1) (layer F.Cu) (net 16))
 (segment (start 16.525 38.135002) (end 16.525 40) (width 1) (layer F.Cu) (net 17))
 (segment (start 13.95 35.560002) (end 16.525 38.135002) (width 1) (layer F.Cu) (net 17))
 (segment (start 13.95 35) (end 13.95 35.560002) (width 1) (layer F.Cu) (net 17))
 (segment (start 16.525 43.135002) (end 16.525 45) (width 1) (layer F.Cu) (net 18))
 (segment (start 13.95 40.560002) (end 16.525 43.135002) (width 1) (layer F.Cu) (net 18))
 (segment (start 13.95 40) (end 13.95 40.560002) (width 1) (layer F.Cu) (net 18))
 (segment (start 16.525 48.964998) (end 16.525 50) (width 1) (layer F.Cu) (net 19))
 (segment (start 13.95 46.389998) (end 16.525 48.964998) (width 1) (layer F.Cu) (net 19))
 (segment (start 13.95 45) (end 13.95 46.389998) (width 1) (layer F.Cu) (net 19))
 (segment (start 16.525 53.135002) (end 16.525 55) (width 1) (layer F.Cu) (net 20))
 (segment (start 13.95 50.560002) (end 16.525 53.135002) (width 1) (layer F.Cu) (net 20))
 (segment (start 13.95 50) (end 13.95 50.560002) (width 1) (layer F.Cu) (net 20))
 (segment (start 16.525 58.964998) (end 16.525 60) (width 1) (layer F.Cu) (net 21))
 (segment (start 13.95 56.389998) (end 16.525 58.964998) (width 1) (layer F.Cu) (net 21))
 (segment (start 13.95 55) (end 13.95 56.389998) (width 1) (layer F.Cu) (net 21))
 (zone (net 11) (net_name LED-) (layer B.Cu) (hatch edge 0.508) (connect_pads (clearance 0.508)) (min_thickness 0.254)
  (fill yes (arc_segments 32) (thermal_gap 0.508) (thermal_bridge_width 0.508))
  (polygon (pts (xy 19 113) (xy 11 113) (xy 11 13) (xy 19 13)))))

